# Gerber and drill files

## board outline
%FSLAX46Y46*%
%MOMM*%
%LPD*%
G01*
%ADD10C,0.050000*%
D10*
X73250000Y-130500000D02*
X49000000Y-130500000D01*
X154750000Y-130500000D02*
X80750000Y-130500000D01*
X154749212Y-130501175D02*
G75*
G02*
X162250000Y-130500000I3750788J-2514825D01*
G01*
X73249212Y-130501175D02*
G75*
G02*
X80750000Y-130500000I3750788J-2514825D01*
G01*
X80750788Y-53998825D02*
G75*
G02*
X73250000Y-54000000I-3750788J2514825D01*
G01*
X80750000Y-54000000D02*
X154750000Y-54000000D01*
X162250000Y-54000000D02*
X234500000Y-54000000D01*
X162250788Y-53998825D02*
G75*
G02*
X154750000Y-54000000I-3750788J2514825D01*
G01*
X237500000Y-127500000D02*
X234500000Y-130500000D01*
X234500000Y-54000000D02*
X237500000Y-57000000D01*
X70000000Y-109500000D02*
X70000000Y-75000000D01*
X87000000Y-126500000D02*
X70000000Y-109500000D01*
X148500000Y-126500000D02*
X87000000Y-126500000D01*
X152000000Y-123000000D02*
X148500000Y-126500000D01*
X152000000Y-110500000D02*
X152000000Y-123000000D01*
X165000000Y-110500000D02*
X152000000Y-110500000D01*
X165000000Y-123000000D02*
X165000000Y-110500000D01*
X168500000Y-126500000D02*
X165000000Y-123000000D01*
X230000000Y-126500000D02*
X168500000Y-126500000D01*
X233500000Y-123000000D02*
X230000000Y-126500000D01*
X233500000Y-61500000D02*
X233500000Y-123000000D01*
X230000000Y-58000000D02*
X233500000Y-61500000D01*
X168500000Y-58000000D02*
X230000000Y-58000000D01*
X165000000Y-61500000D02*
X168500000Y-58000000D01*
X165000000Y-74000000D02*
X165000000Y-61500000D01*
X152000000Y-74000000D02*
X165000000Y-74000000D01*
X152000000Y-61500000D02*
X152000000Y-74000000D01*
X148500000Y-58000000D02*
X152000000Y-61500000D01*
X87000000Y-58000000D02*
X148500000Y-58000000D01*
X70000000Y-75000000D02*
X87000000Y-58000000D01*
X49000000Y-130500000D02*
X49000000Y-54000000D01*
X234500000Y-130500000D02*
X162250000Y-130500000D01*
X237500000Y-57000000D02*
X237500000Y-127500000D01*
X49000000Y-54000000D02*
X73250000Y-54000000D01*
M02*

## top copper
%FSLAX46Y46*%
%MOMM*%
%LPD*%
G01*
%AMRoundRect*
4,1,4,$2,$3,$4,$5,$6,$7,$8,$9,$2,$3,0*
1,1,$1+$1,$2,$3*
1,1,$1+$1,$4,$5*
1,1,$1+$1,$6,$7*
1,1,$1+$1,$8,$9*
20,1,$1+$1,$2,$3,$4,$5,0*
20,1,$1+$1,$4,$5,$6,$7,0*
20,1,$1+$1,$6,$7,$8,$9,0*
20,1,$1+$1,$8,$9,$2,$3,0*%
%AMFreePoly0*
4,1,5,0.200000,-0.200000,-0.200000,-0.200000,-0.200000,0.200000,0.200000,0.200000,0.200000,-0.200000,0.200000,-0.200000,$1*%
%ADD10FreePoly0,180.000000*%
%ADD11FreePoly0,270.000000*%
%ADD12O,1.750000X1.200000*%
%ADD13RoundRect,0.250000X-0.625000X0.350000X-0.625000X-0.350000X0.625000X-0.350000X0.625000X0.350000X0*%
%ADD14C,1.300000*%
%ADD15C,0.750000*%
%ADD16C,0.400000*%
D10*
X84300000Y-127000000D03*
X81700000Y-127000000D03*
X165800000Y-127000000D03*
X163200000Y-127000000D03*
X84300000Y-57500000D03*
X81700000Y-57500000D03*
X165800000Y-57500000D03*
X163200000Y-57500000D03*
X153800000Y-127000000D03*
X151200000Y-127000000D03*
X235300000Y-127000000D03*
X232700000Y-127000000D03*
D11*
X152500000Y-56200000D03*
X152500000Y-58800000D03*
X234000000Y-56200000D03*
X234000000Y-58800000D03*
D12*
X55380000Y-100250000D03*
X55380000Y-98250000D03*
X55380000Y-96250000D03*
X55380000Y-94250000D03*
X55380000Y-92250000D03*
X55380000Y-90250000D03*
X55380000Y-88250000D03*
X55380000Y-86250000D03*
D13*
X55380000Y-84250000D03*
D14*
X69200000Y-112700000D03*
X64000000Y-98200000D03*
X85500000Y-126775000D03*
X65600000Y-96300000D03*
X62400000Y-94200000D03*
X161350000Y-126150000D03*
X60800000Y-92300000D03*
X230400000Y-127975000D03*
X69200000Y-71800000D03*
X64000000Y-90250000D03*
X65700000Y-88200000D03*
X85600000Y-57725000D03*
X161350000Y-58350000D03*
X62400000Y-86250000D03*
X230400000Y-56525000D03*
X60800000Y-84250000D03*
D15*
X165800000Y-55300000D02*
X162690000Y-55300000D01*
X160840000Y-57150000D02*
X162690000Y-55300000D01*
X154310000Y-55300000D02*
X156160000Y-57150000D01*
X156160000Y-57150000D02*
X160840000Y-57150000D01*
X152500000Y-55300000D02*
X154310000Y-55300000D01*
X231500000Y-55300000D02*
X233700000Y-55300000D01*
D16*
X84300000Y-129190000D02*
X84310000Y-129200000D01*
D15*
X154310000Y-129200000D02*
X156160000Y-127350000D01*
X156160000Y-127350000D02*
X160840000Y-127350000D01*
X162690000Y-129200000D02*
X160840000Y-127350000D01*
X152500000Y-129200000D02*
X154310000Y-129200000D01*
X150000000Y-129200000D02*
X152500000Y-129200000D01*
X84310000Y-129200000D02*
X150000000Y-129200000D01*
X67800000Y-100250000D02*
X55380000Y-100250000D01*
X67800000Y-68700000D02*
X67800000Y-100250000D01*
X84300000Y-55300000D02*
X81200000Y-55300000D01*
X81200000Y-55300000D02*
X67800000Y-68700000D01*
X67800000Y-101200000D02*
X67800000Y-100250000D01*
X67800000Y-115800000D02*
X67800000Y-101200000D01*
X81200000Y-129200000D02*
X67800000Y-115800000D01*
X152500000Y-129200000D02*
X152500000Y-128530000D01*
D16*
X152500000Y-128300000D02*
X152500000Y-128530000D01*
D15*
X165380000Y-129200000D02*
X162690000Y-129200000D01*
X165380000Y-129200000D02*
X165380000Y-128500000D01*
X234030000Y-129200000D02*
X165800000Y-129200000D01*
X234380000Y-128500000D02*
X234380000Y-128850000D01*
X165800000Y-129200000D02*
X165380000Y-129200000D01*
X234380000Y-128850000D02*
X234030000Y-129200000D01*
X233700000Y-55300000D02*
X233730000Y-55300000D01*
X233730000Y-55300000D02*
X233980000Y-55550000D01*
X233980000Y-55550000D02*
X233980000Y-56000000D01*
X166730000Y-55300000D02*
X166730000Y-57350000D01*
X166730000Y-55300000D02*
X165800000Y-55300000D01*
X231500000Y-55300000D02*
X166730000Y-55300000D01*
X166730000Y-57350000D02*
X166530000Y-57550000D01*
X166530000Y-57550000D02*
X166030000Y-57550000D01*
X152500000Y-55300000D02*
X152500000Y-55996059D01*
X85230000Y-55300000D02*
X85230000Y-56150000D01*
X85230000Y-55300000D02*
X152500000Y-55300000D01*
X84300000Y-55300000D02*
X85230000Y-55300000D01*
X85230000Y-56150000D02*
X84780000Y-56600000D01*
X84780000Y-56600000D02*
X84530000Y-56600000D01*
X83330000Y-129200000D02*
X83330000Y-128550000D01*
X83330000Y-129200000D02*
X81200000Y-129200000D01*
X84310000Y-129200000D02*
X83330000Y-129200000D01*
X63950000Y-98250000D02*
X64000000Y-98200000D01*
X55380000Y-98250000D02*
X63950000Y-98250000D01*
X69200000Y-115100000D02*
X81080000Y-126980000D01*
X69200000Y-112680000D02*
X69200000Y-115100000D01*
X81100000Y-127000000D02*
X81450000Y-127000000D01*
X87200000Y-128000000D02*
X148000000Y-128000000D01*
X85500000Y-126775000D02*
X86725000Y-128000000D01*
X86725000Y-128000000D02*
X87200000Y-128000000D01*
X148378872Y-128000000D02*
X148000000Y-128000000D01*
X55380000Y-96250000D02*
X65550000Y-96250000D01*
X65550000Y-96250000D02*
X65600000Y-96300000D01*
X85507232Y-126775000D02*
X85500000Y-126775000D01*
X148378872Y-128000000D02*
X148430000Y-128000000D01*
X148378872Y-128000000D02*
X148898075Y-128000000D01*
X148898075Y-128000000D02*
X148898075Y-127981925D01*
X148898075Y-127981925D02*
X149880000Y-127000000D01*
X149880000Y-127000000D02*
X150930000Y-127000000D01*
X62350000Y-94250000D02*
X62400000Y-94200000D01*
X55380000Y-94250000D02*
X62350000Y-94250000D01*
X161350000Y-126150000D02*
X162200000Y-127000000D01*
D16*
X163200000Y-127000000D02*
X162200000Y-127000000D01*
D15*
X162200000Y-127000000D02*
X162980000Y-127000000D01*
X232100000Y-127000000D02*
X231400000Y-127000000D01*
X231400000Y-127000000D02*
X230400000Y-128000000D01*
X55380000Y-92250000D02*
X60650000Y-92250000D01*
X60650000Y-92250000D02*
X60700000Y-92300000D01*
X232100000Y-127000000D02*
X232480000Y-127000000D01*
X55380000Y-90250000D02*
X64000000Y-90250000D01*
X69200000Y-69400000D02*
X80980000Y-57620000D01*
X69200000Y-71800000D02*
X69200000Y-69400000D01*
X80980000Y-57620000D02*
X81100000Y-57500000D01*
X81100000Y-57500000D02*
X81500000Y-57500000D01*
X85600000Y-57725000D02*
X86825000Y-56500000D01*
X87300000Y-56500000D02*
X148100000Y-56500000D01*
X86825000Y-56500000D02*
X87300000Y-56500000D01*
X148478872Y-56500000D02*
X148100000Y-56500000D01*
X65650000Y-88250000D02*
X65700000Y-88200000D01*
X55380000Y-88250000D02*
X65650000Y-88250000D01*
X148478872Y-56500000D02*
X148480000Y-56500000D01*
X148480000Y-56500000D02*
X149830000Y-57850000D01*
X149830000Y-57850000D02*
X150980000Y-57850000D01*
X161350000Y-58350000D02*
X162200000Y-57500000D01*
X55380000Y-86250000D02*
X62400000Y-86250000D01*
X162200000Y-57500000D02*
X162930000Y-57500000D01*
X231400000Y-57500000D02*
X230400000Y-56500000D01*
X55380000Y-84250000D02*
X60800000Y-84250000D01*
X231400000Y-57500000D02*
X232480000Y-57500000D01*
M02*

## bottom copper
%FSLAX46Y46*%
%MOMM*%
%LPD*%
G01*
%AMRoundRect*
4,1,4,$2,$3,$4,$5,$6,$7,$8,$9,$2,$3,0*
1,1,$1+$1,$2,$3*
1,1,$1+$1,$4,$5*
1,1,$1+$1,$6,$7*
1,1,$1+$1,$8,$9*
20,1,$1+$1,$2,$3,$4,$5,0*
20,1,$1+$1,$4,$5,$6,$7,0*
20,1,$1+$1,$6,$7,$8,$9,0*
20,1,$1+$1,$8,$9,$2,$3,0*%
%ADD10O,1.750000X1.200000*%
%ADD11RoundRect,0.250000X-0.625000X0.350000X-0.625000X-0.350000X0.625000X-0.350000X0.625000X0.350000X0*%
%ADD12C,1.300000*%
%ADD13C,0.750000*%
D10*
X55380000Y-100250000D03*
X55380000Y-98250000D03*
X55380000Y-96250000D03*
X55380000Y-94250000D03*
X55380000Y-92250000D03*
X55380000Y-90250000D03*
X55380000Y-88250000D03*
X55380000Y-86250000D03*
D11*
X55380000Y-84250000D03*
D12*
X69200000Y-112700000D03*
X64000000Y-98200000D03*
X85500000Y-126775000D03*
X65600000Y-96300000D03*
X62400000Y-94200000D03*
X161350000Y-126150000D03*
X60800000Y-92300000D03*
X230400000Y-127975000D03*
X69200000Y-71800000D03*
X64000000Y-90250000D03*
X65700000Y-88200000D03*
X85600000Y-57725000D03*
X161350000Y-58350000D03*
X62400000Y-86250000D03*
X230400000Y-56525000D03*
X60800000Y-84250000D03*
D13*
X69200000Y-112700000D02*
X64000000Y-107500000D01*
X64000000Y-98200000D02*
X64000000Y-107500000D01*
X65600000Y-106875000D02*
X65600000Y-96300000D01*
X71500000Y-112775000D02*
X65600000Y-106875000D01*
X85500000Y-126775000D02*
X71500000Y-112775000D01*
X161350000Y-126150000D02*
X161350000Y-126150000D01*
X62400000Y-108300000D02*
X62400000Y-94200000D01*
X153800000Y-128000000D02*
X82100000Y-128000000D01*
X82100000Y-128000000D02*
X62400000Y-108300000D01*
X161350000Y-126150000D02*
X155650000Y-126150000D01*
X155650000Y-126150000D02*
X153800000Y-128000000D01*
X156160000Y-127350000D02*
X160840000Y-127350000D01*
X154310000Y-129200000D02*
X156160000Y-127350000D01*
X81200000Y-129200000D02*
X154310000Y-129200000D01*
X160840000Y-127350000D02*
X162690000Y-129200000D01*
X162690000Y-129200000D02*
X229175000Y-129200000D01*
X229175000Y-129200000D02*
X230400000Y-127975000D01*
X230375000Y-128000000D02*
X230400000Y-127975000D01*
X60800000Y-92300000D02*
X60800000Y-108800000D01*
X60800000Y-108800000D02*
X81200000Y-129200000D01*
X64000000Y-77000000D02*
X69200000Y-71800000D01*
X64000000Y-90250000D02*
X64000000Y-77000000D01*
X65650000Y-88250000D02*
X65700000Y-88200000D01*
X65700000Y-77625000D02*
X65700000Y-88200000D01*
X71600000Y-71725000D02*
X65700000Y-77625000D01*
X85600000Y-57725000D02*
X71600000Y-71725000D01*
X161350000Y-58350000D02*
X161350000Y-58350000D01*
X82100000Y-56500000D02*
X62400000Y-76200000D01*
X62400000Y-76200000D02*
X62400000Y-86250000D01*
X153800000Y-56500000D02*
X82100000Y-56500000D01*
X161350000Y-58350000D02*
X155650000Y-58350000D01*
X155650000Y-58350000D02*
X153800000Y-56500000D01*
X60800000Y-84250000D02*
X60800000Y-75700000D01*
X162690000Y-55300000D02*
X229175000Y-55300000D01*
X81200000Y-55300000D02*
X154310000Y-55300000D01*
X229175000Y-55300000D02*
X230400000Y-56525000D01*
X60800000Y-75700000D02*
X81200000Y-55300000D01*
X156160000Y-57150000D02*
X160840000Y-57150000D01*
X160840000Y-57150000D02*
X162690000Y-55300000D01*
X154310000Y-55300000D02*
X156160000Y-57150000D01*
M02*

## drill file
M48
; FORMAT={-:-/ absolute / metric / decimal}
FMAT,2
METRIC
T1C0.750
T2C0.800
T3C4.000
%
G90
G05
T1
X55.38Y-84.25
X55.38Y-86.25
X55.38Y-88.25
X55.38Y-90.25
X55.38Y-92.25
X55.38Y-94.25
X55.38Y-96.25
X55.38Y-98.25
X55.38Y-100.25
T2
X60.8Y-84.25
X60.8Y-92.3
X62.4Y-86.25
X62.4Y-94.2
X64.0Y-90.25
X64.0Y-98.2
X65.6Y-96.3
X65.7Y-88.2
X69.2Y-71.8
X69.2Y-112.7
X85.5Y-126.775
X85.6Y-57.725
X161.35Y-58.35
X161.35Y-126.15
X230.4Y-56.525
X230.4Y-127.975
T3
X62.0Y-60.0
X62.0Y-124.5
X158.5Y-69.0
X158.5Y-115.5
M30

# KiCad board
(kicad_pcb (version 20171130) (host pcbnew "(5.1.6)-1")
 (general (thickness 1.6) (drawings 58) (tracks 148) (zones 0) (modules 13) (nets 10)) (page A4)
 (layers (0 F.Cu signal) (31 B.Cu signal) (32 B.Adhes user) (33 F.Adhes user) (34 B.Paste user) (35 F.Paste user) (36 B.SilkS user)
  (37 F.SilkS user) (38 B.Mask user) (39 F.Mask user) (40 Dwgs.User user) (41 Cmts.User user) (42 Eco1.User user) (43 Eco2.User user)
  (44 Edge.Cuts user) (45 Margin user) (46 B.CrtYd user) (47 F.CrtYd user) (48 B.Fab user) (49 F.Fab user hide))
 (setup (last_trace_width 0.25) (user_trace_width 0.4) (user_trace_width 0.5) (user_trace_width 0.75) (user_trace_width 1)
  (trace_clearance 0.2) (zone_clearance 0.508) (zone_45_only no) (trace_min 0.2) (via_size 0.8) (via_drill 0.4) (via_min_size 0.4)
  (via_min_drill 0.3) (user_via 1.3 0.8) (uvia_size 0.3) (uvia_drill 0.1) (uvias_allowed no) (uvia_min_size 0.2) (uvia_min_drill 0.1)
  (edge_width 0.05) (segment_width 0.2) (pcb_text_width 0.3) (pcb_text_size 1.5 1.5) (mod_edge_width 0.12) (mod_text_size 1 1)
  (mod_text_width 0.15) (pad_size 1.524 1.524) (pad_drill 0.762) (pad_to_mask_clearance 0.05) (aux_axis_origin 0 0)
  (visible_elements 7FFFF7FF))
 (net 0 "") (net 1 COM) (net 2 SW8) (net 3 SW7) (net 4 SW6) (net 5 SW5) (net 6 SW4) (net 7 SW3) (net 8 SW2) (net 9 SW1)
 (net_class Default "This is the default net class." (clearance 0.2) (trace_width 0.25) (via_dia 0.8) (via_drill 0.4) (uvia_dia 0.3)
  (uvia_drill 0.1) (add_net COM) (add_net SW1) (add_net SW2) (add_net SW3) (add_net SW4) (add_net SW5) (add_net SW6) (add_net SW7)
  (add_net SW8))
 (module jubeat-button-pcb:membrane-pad (layer F.Cu) (at 83 127 180)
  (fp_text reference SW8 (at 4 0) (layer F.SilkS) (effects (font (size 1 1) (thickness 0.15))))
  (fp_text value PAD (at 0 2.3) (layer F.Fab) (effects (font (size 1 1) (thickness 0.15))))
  (pad 1 smd custom (at -1.3 0 180) (size 0.4 0.4) (layers F.Cu F.Paste F.Mask) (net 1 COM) (zone_connect 0)
   (options (clearance outline) (anchor rect)) (primitives))
  (pad 2 smd custom (at 1.3 0 180) (size 0.4 0.4) (layers F.Cu F.Paste F.Mask) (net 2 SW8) (zone_connect 0)
   (options (clearance outline) (anchor rect)) (primitives)))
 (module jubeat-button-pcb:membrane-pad (layer F.Cu) (at 164.5 127 180)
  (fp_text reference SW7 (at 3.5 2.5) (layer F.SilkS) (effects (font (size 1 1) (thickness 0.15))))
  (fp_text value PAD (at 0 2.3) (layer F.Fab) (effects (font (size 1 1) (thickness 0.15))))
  (pad 1 smd custom (at -1.3 0 180) (size 0.4 0.4) (layers F.Cu F.Paste F.Mask) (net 1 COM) (zone_connect 0)
   (options (clearance outline) (anchor rect)) (primitives))
  (pad 2 smd custom (at 1.3 0 180) (size 0.4 0.4) (layers F.Cu F.Paste F.Mask) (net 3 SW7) (zone_connect 0)
   (options (clearance outline) (anchor rect)) (primitives)))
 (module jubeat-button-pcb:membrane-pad (layer F.Cu) (at 83 57.5 180)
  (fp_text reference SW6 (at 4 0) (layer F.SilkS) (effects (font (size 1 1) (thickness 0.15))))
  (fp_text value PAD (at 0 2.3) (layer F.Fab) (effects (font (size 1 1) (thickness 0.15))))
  (pad 1 smd custom (at -1.3 0 180) (size 0.4 0.4) (layers F.Cu F.Paste F.Mask) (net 1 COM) (zone_connect 0)
   (options (clearance outline) (anchor rect)) (primitives))
  (pad 2 smd custom (at 1.3 0 180) (size 0.4 0.4) (layers F.Cu F.Paste F.Mask) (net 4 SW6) (zone_connect 0)
   (options (clearance outline) (anchor rect)) (primitives)))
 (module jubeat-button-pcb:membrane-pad (layer F.Cu) (at 164.5 57.5 180)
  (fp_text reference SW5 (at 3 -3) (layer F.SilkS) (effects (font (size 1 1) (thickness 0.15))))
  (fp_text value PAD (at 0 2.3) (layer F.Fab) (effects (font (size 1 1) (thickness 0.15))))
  (pad 1 smd custom (at -1.3 0 180) (size 0.4 0.4) (layers F.Cu F.Paste F.Mask) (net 1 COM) (zone_connect 0)
   (options (clearance outline) (anchor rect)) (primitives))
  (pad 2 smd custom (at 1.3 0 180) (size 0.4 0.4) (layers F.Cu F.Paste F.Mask) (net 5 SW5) (zone_connect 0)
   (options (clearance outline) (anchor rect)) (primitives)))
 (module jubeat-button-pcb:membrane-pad (layer F.Cu) (at 152.5 127 180)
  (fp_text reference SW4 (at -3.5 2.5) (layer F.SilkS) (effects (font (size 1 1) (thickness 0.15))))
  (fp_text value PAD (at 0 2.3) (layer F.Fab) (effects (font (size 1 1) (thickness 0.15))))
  (pad 1 smd custom (at -1.3 0 180) (size 0.4 0.4) (layers F.Cu F.Paste F.Mask) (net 1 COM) (zone_connect 0)
   (options (clearance outline) (anchor rect)) (primitives))
  (pad 2 smd custom (at 1.3 0 180) (size 0.4 0.4) (layers F.Cu F.Paste F.Mask) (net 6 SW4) (zone_connect 0)
   (options (clearance outline) (anchor rect)) (primitives)))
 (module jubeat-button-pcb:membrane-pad (layer F.Cu) (at 234 127 180)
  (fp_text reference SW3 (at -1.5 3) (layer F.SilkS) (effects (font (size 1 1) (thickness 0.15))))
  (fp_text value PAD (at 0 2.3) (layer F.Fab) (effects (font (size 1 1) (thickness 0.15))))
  (pad 1 smd custom (at -1.3 0 180) (size 0.4 0.4) (layers F.Cu F.Paste F.Mask) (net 1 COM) (zone_connect 0)
   (options (clearance outline) (anchor rect)) (primitives))
  (pad 2 smd custom (at 1.3 0 180) (size 0.4 0.4) (layers F.Cu F.Paste F.Mask) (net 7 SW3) (zone_connect 0)
   (options (clearance outline) (anchor rect)) (primitives)))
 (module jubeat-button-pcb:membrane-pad (layer F.Cu) (at 152.5 57.5 270)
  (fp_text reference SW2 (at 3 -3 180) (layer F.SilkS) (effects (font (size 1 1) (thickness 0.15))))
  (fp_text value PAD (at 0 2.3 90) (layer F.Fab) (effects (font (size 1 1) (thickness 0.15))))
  (pad 1 smd custom (at -1.3 0 270) (size 0.4 0.4) (layers F.Cu F.Paste F.Mask) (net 1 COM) (zone_connect 0)
   (options (clearance outline) (anchor rect)) (primitives))
  (pad 2 smd custom (at 1.3 0 270) (size 0.4 0.4) (layers F.Cu F.Paste F.Mask) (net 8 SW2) (zone_connect 0)
   (options (clearance outline) (anchor rect)) (primitives)))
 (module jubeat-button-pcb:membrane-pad (layer F.Cu) (at 234 57.5 270)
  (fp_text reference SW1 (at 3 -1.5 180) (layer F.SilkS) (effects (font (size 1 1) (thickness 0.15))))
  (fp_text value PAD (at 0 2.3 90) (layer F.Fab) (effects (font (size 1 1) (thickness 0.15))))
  (pad 1 smd custom (at -1.3 0 270) (size 0.4 0.4) (layers F.Cu F.Paste F.Mask) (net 1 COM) (zone_connect 0)
   (options (clearance outline) (anchor rect)) (primitives))
  (pad 2 smd custom (at 1.3 0 270) (size 0.4 0.4) (layers F.Cu F.Paste F.Mask) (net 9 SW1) (zone_connect 0)
   (options (clearance outline) (anchor rect)) (primitives)))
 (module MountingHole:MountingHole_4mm (layer F.Cu) (at 158.5 115.5)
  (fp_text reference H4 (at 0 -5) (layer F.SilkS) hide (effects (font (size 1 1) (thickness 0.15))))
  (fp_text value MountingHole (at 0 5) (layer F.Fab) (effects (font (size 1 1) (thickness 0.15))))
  (pad 1 np_thru_hole circle (at 0 0) (size 4 4) (drill 4) (layers *.Cu *.Mask)))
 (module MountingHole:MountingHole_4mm (layer F.Cu) (at 158.5 69)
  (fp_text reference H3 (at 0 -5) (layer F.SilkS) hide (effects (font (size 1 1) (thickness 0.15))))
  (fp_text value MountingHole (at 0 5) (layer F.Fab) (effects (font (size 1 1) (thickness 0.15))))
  (pad 1 np_thru_hole circle (at 0 0) (size 4 4) (drill 4) (layers *.Cu *.Mask)))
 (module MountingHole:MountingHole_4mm (layer F.Cu) (at 62 124.5)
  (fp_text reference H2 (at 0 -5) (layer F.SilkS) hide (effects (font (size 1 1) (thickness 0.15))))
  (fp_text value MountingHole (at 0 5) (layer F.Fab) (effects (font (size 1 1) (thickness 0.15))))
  (pad 1 np_thru_hole circle (at 0 0) (size 4 4) (drill 4) (layers *.Cu *.Mask)))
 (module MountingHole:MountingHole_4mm (layer F.Cu) (at 62 60)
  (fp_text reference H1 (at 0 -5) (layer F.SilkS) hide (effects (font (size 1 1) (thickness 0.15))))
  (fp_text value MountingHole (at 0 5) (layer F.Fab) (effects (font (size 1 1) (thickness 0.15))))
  (pad 1 np_thru_hole circle (at 0 0) (size 4 4) (drill 4) (layers *.Cu *.Mask)))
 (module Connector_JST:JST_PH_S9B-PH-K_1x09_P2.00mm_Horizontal (layer F.Cu) (at 55.38 84.25 270)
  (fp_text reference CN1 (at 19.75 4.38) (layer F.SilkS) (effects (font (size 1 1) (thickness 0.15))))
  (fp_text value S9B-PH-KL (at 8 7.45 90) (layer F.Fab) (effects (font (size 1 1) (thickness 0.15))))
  (pad 9 thru_hole oval (at 16 0 270) (size 1.2 1.75) (drill 0.75) (layers *.Cu *.Mask) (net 1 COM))
  (pad 8 thru_hole oval (at 14 0 270) (size 1.2 1.75) (drill 0.75) (layers *.Cu *.Mask) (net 2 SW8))
  (pad 7 thru_hole oval (at 12 0 270) (size 1.2 1.75) (drill 0.75) (layers *.Cu *.Mask) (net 6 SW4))
  (pad 6 thru_hole oval (at 10 0 270) (size 1.2 1.75) (drill 0.75) (layers *.Cu *.Mask) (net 3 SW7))
  (pad 5 thru_hole oval (at 8 0 270) (size 1.2 1.75) (drill 0.75) (layers *.Cu *.Mask) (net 7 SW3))
  (pad 4 thru_hole oval (at 6 0 270) (size 1.2 1.75) (drill 0.75) (layers *.Cu *.Mask) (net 4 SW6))
  (pad 3 thru_hole oval (at 4 0 270) (size 1.2 1.75) (drill 0.75) (layers *.Cu *.Mask) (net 8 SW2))
  (pad 2 thru_hole oval (at 2 0 270) (size 1.2 1.75) (drill 0.75) (layers *.Cu *.Mask) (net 5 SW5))
  (pad 1 thru_hole roundrect (at 0 0 270) (size 1.2 1.75) (drill 0.75) (layers *.Cu *.Mask) (roundrect_rratio 0.208333) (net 9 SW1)))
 (gr_line (start 73.25 130.5) (end 49 130.5) (layer Edge.Cuts) (width 0.05))
 (gr_line (start 154.75 130.5) (end 80.75 130.5) (layer Edge.Cuts) (width 0.05))
 (gr_arc (start 158.5 133.016) (end 162.25 130.5) (angle -112.3) (layer Edge.Cuts) (width 0.05))
 (gr_arc (start 77 133.016) (end 80.75 130.5) (angle -112.3) (layer Edge.Cuts) (width 0.05))
 (gr_arc (start 77 51.484) (end 73.25 54) (angle -112.3) (layer Edge.Cuts) (width 0.05))
 (gr_line (start 80.75 54) (end 154.75 54) (layer Edge.Cuts) (width 0.05))
 (gr_line (start 162.25 54) (end 234.5 54) (layer Edge.Cuts) (width 0.05))
 (gr_arc (start 158.5 51.484) (end 154.75 54) (angle -112.3) (layer Edge.Cuts) (width 0.05))
 (gr_line (start 237.5 127.5) (end 234.5 130.5) (layer Edge.Cuts) (width 0.05))
 (gr_line (start 234.5 54) (end 237.5 57) (layer Edge.Cuts) (width 0.05))
 (gr_line (start 70 109.5) (end 70 75) (layer Edge.Cuts) (width 0.05))
 (gr_line (start 87 126.5) (end 70 109.5) (layer Edge.Cuts) (width 0.05))
 (gr_line (start 148.5 126.5) (end 87 126.5) (layer Edge.Cuts) (width 0.05))
 (gr_line (start 152 123) (end 148.5 126.5) (layer Edge.Cuts) (width 0.05))
 (gr_line (start 152 110.5) (end 152 123) (layer Edge.Cuts) (width 0.05))
 (gr_line (start 165 110.5) (end 152 110.5) (layer Edge.Cuts) (width 0.05))
 (gr_line (start 165 123) (end 165 110.5) (layer Edge.Cuts) (width 0.05))
 (gr_line (start 168.5 126.5) (end 165 123) (layer Edge.Cuts) (width 0.05))
 (gr_line (start 230 126.5) (end 168.5 126.5) (layer Edge.Cuts) (width 0.05))
 (gr_line (start 233.5 123) (end 230 126.5) (layer Edge.Cuts) (width 0.05))
 (gr_line (start 233.5 61.5) (end 233.5 123) (layer Edge.Cuts) (width 0.05))
 (gr_line (start 230 58) (end 233.5 61.5) (layer Edge.Cuts) (width 0.05))
 (gr_line (start 168.5 58) (end 230 58) (layer Edge.Cuts) (width 0.05))
 (gr_line (start 165 61.5) (end 168.5 58) (layer Edge.Cuts) (width 0.05))
 (gr_line (start 165 74) (end 165 61.5) (layer Edge.Cuts) (width 0.05))
 (gr_line (start 152 74) (end 165 74) (layer Edge.Cuts) (width 0.05))
 (gr_line (start 152 61.5) (end 152 74) (layer Edge.Cuts) (width 0.05))
 (gr_line (start 148.5 58) (end 152 61.5) (layer Edge.Cuts) (width 0.05))
 (gr_line (start 87 58) (end 148.5 58) (layer Edge.Cuts) (width 0.05))
 (gr_line (start 70 75) (end 87 58) (layer Edge.Cuts) (width 0.05))
 (gr_line (start 49 130.5) (end 49 54) (layer Edge.Cuts) (width 0.05))
 (gr_line (start 234.5 130.5) (end 162.25 130.5) (layer Edge.Cuts) (width 0.05))
 (gr_line (start 237.5 57) (end 237.5 127.5) (layer Edge.Cuts) (width 0.05))
 (gr_line (start 49 54) (end 73.25 54) (layer Edge.Cuts) (width 0.05))
 (segment (start 165.8 55.3) (end 162.69 55.3) (width 0.75) (layer F.Cu) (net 1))
 (segment (start 160.84 57.15) (end 162.69 55.3) (width 0.75) (layer F.Cu) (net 1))
 (segment (start 154.31 55.3) (end 156.16 57.15) (width 0.75) (layer F.Cu) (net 1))
 (segment (start 156.16 57.15) (end 160.84 57.15) (width 0.75) (layer F.Cu) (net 1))
 (segment (start 152.5 55.3) (end 154.31 55.3) (width 0.75) (layer F.Cu) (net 1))
 (segment (start 231.5 55.3) (end 233.7 55.3) (width 0.75) (layer F.Cu) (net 1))
 (segment (start 84.3 129.19) (end 84.31 129.2) (width 0.4) (layer F.Cu) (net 1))
 (segment (start 154.31 129.2) (end 156.16 127.35) (width 0.75) (layer F.Cu) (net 1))
 (segment (start 156.16 127.35) (end 160.84 127.35) (width 0.75) (layer F.Cu) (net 1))
 (segment (start 162.69 129.2) (end 160.84 127.35) (width 0.75) (layer F.Cu) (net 1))
 (segment (start 152.5 129.2) (end 154.31 129.2) (width 0.75) (layer F.Cu) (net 1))
 (segment (start 150 129.2) (end 152.5 129.2) (width 0.75) (layer F.Cu) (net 1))
 (segment (start 84.31 129.2) (end 150 129.2) (width 0.75) (layer F.Cu) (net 1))
 (segment (start 67.8 100.25) (end 55.38 100.25) (width 0.75) (layer F.Cu) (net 1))
 (segment (start 67.8 68.7) (end 67.8 100.25) (width 0.75) (layer F.Cu) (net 1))
 (segment (start 84.3 55.3) (end 81.2 55.3) (width 0.75) (layer F.Cu) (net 1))
 (segment (start 81.2 55.3) (end 67.8 68.7) (width 0.75) (layer F.Cu) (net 1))
 (segment (start 67.8 101.2) (end 67.8 100.25) (width 0.75) (layer F.Cu) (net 1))
 (segment (start 67.8 115.8) (end 67.8 101.2) (width 0.75) (layer F.Cu) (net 1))
 (segment (start 81.2 129.2) (end 67.8 115.8) (width 0.75) (layer F.Cu) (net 1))
 (segment (start 152.5 129.2) (end 152.5 128.53) (width 0.75) (layer F.Cu) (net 1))
 (segment (start 152.5 128.3) (end 152.5 128.53) (width 0.4) (layer F.Cu) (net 1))
 (segment (start 165.38 129.2) (end 162.69 129.2) (width 0.75) (layer F.Cu) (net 1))
 (segment (start 165.38 129.2) (end 165.38 128.5) (width 0.75) (layer F.Cu) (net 1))
 (segment (start 234.03 129.2) (end 165.8 129.2) (width 0.75) (layer F.Cu) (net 1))
 (segment (start 234.38 128.5) (end 234.38 128.85) (width 0.75) (layer F.Cu) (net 1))
 (segment (start 165.8 129.2) (end 165.38 129.2) (width 0.75) (layer F.Cu) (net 1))
 (segment (start 234.38 128.85) (end 234.03 129.2) (width 0.75) (layer F.Cu) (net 1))
 (segment (start 233.7 55.3) (end 233.73 55.3) (width 0.75) (layer F.Cu) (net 1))
 (segment (start 233.73 55.3) (end 233.98 55.55) (width 0.75) (layer F.Cu) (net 1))
 (segment (start 233.98 55.55) (end 233.98 56) (width 0.75) (layer F.Cu) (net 1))
 (segment (start 166.73 55.3) (end 166.73 57.35) (width 0.75) (layer F.Cu) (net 1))
 (segment (start 166.73 55.3) (end 165.8 55.3) (width 0.75) (layer F.Cu) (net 1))
 (segment (start 231.5 55.3) (end 166.73 55.3) (width 0.75) (layer F.Cu) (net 1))
 (segment (start 166.73 57.35) (end 166.53 57.55) (width 0.75) (layer F.Cu) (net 1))
 (segment (start 166.53 57.55) (end 166.03 57.55) (width 0.75) (layer F.Cu) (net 1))
 (segment (start 152.5 55.3) (end 152.5 55.996059) (width 0.75) (layer F.Cu) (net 1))
 (segment (start 85.23 55.3) (end 85.23 56.15) (width 0.75) (layer F.Cu) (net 1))
 (segment (start 85.23 55.3) (end 152.5 55.3) (width 0.75) (layer F.Cu) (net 1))
 (segment (start 84.3 55.3) (end 85.23 55.3) (width 0.75) (layer F.Cu) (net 1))
 (segment (start 85.23 56.15) (end 84.78 56.6) (width 0.75) (layer F.Cu) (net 1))
 (segment (start 84.78 56.6) (end 84.53 56.6) (width 0.75) (layer F.Cu) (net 1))
 (segment (start 83.33 129.2) (end 83.33 128.55) (width 0.75) (layer F.Cu) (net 1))
 (segment (start 83.33 129.2) (end 81.2 129.2) (width 0.75) (layer F.Cu) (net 1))
 (segment (start 84.31 129.2) (end 83.33 129.2) (width 0.75) (layer F.Cu) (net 1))
 (via (at 69.2 112.7) (size 1.3) (drill 0.8) (layers F.Cu B.Cu) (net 2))
 (via (at 64 98.2) (size 1.3) (drill 0.8) (layers F.Cu B.Cu) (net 2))
 (segment (start 69.2 112.7) (end 64 107.5) (width 0.75) (layer B.Cu) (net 2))
 (segment (start 63.95 98.25) (end 64 98.2) (width 0.75) (layer F.Cu) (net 2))
 (segment (start 55.38 98.25) (end 63.95 98.25) (width 0.75) (layer F.Cu) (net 2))
 (segment (start 64 98.2) (end 64 107.5) (width 0.75) (layer B.Cu) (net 2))
 (segment (start 69.2 115.1) (end 81.08 126.98) (width 0.75) (layer F.Cu) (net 2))
 (segment (start 69.2 112.68) (end 69.2 115.1) (width 0.75) (layer F.Cu) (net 2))
 (segment (start 81.1 127) (end 81.45 127) (width 0.75) (layer F.Cu) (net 2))
 (segment (start 87.2 128) (end 148 128) (width 0.75) (layer F.Cu) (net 6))
 (segment (start 85.5 126.775) (end 86.725 128) (width 0.75) (layer F.Cu) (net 6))
 (segment (start 86.725 128) (end 87.2 128) (width 0.75) (layer F.Cu) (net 6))
 (segment (start 148.378872 128) (end 148 128) (width 0.75) (layer F.Cu) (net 6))
 (via (at 85.5 126.775) (size 1.3) (drill 0.8) (layers F.Cu B.Cu) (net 6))
 (segment (start 55.38 96.25) (end 65.55 96.25) (width 0.75) (layer F.Cu) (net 6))
 (segment (start 65.55 96.25) (end 65.6 96.3) (width 0.75) (layer F.Cu) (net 6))
 (segment (start 65.6 106.875) (end 65.6 96.3) (width 0.75) (layer B.Cu) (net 6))
 (segment (start 71.5 112.775) (end 65.6 106.875) (width 0.75) (layer B.Cu) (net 6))
 (via (at 65.6 96.3) (size 1.3) (drill 0.8) (layers F.Cu B.Cu) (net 6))
 (segment (start 85.5 126.775) (end 71.5 112.775) (width 0.75) (layer B.Cu) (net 6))
 (segment (start 85.507232 126.775) (end 85.5 126.775) (width 0.75) (layer F.Cu) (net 6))
 (segment (start 148.378872 128) (end 148.43 128) (width 0.75) (layer F.Cu) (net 6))
 (segment (start 148.378872 128) (end 148.898075 128) (width 0.75) (layer F.Cu) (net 6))
 (segment (start 148.898075 128) (end 148.898075 127.981925) (width 0.75) (layer F.Cu) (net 6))
 (segment (start 148.898075 127.981925) (end 149.88 127) (width 0.75) (layer F.Cu) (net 6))
 (segment (start 149.88 127) (end 150.93 127) (width 0.75) (layer F.Cu) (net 6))
 (via (at 62.4 94.2) (size 1.3) (drill 0.8) (layers F.Cu B.Cu) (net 3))
 (segment (start 62.35 94.25) (end 62.4 94.2) (width 0.75) (layer F.Cu) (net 3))
 (segment (start 55.38 94.25) (end 62.35 94.25) (width 0.75) (layer F.Cu) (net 3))
 (segment (start 161.35 126.15) (end 161.35 126.15) (width 0.75) (layer B.Cu) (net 3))
 (via (at 161.35 126.15) (size 1.3) (drill 0.8) (layers F.Cu B.Cu) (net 3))
 (segment (start 161.35 126.15) (end 162.2 127) (width 0.75) (layer F.Cu) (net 3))
 (segment (start 163.2 127) (end 162.2 127) (width 0.4) (layer F.Cu) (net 3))
 (segment (start 62.4 108.3) (end 62.4 94.2) (width 0.75) (layer B.Cu) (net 3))
 (segment (start 153.8 128) (end 82.1 128) (width 0.75) (layer B.Cu) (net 3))
 (segment (start 82.1 128) (end 62.4 108.3) (width 0.75) (layer B.Cu) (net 3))
 (segment (start 161.35 126.15) (end 155.65 126.15) (width 0.75) (layer B.Cu) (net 3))
 (segment (start 155.65 126.15) (end 153.8 128) (width 0.75) (layer B.Cu) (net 3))
 (segment (start 162.2 127) (end 162.98 127) (width 0.75) (layer F.Cu) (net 3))
 (segment (start 232.1 127) (end 231.4 127) (width 0.75) (layer F.Cu) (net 7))
 (segment (start 231.4 127) (end 230.4 128) (width 0.75) (layer F.Cu) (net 7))
 (via (at 60.8 92.3) (size 1.3) (drill 0.8) (layers F.Cu B.Cu) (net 7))
 (segment (start 156.16 127.35) (end 160.84 127.35) (width 0.75) (layer B.Cu) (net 7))
 (segment (start 154.31 129.2) (end 156.16 127.35) (width 0.75) (layer B.Cu) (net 7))
 (segment (start 81.2 129.2) (end 154.31 129.2) (width 0.75) (layer B.Cu) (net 7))
 (segment (start 160.84 127.35) (end 162.69 129.2) (width 0.75) (layer B.Cu) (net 7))
 (segment (start 162.69 129.2) (end 229.175 129.2) (width 0.75) (layer B.Cu) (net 7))
 (segment (start 229.175 129.2) (end 230.4 127.975) (width 0.75) (layer B.Cu) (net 7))
 (segment (start 230.375 128) (end 230.4 127.975) (width 0.75) (layer B.Cu) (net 7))
 (via (at 230.4 127.975) (size 1.3) (drill 0.8) (layers F.Cu B.Cu) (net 7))
 (segment (start 55.38 92.25) (end 60.65 92.25) (width 0.75) (layer F.Cu) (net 7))
 (segment (start 60.65 92.25) (end 60.7 92.3) (width 0.75) (layer F.Cu) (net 7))
 (segment (start 60.8 92.3) (end 60.8 108.8) (width 0.75) (layer B.Cu) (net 7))
 (segment (start 60.8 108.8) (end 81.2 129.2) (width 0.75) (layer B.Cu) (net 7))
 (segment (start 232.1 127) (end 232.48 127) (width 0.75) (layer F.Cu) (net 7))
 (via (at 69.2 71.8) (size 1.3) (drill 0.8) (layers F.Cu B.Cu) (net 4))
 (via (at 64 90.25) (size 1.3) (drill 0.8) (layers F.Cu B.Cu) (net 4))
 (segment (start 55.38 90.25) (end 64 90.25) (width 0.75) (layer F.Cu) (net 4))
 (segment (start 64 77) (end 69.2 71.8) (width 0.75) (layer B.Cu) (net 4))
 (segment (start 64 90.25) (end 64 77) (width 0.75) (layer B.Cu) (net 4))
 (segment (start 69.2 69.4) (end 80.98 57.62) (width 0.75) (layer F.Cu) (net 4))
 (segment (start 69.2 71.8) (end 69.2 69.4) (width 0.75) (layer F.Cu) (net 4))
 (segment (start 80.98 57.62) (end 81.1 57.5) (width 0.75) (layer F.Cu) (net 4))
 (segment (start 81.1 57.5) (end 81.5 57.5) (width 0.75) (layer F.Cu) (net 4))
 (via (at 65.7 88.2) (size 1.3) (drill 0.8) (layers F.Cu B.Cu) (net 8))
 (segment (start 85.6 57.725) (end 86.825 56.5) (width 0.75) (layer F.Cu) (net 8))
 (segment (start 87.3 56.5) (end 148.1 56.5) (width 0.75) (layer F.Cu) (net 8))
 (segment (start 86.825 56.5) (end 87.3 56.5) (width 0.75) (layer F.Cu) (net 8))
 (via (at 85.6 57.725) (size 1.3) (drill 0.8) (layers F.Cu B.Cu) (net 8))
 (segment (start 65.65 88.25) (end 65.7 88.2) (width 0.75) (layer B.Cu) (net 8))
 (segment (start 65.7 77.625) (end 65.7 88.2) (width 0.75) (layer B.Cu) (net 8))
 (segment (start 71.6 71.725) (end 65.7 77.625) (width 0.75) (layer B.Cu) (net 8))
 (segment (start 85.6 57.725) (end 71.6 71.725) (width 0.75) (layer B.Cu) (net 8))
 (segment (start 148.478872 56.5) (end 148.1 56.5) (width 0.75) (layer F.Cu) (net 8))
 (segment (start 65.65 88.25) (end 65.7 88.2) (width 0.75) (layer F.Cu) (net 8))
 (segment (start 55.38 88.25) (end 65.65 88.25) (width 0.75) (layer F.Cu) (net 8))
 (segment (start 148.478872 56.5) (end 148.48 56.5) (width 0.75) (layer F.Cu) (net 8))
 (segment (start 148.48 56.5) (end 149.83 57.85) (width 0.75) (layer F.Cu) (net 8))
 (segment (start 149.83 57.85) (end 150.98 57.85) (width 0.75) (layer F.Cu) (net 8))
 (segment (start 161.35 58.35) (end 161.35 58.35) (width 0.75) (layer B.Cu) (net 5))
 (via (at 161.35 58.35) (size 1.3) (drill 0.8) (layers F.Cu B.Cu) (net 5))
 (segment (start 161.35 58.35) (end 162.2 57.5) (width 0.75) (layer F.Cu) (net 5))
 (via (at 62.4 86.25) (size 1.3) (drill 0.8) (layers F.Cu B.Cu) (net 5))
 (segment (start 55.38 86.25) (end 62.4 86.25) (width 0.75) (layer F.Cu) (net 5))
 (segment (start 82.1 56.5) (end 62.4 76.2) (width 0.75) (layer B.Cu) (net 5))
 (segment (start 62.4 76.2) (end 62.4 86.25) (width 0.75) (layer B.Cu) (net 5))
 (segment (start 153.8 56.5) (end 82.1 56.5) (width 0.75) (layer B.Cu) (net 5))
 (segment (start 161.35 58.35) (end 155.65 58.35) (width 0.75) (layer B.Cu) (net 5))
 (segment (start 155.65 58.35) (end 153.8 56.5) (width 0.75) (layer B.Cu) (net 5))
 (segment (start 162.2 57.5) (end 162.93 57.5) (width 0.75) (layer F.Cu) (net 5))
 (via (at 230.4 56.525) (size 1.3) (drill 0.8) (layers F.Cu B.Cu) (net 9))
 (segment (start 231.4 57.5) (end 230.4 56.5) (width 0.75) (layer F.Cu) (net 9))
 (via (at 60.8 84.25) (size 1.3) (drill 0.8) (layers F.Cu B.Cu) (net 9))
 (segment (start 55.38 84.25) (end 60.8 84.25) (width 0.75) (layer F.Cu) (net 9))
 (segment (start 60.8 84.25) (end 60.8 75.7) (width 0.75) (layer B.Cu) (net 9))
 (segment (start 162.69 55.3) (end 229.175 55.3) (width 0.75) (layer B.Cu) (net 9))
 (segment (start 81.2 55.3) (end 154.31 55.3) (width 0.75) (layer B.Cu) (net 9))
 (segment (start 229.175 55.3) (end 230.4 56.525) (width 0.75) (layer B.Cu) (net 9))
 (segment (start 60.8 75.7) (end 81.2 55.3) (width 0.75) (layer B.Cu) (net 9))
 (segment (start 156.16 57.15) (end 160.84 57.15) (width 0.75) (layer B.Cu) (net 9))
 (segment (start 160.84 57.15) (end 162.69 55.3) (width 0.75) (layer B.Cu) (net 9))
 (segment (start 154.31 55.3) (end 156.16 57.15) (width 0.75) (layer B.Cu) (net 9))
 (segment (start 231.4 57.5) (end 232.48 57.5) (width 0.75) (layer F.Cu) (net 9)))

